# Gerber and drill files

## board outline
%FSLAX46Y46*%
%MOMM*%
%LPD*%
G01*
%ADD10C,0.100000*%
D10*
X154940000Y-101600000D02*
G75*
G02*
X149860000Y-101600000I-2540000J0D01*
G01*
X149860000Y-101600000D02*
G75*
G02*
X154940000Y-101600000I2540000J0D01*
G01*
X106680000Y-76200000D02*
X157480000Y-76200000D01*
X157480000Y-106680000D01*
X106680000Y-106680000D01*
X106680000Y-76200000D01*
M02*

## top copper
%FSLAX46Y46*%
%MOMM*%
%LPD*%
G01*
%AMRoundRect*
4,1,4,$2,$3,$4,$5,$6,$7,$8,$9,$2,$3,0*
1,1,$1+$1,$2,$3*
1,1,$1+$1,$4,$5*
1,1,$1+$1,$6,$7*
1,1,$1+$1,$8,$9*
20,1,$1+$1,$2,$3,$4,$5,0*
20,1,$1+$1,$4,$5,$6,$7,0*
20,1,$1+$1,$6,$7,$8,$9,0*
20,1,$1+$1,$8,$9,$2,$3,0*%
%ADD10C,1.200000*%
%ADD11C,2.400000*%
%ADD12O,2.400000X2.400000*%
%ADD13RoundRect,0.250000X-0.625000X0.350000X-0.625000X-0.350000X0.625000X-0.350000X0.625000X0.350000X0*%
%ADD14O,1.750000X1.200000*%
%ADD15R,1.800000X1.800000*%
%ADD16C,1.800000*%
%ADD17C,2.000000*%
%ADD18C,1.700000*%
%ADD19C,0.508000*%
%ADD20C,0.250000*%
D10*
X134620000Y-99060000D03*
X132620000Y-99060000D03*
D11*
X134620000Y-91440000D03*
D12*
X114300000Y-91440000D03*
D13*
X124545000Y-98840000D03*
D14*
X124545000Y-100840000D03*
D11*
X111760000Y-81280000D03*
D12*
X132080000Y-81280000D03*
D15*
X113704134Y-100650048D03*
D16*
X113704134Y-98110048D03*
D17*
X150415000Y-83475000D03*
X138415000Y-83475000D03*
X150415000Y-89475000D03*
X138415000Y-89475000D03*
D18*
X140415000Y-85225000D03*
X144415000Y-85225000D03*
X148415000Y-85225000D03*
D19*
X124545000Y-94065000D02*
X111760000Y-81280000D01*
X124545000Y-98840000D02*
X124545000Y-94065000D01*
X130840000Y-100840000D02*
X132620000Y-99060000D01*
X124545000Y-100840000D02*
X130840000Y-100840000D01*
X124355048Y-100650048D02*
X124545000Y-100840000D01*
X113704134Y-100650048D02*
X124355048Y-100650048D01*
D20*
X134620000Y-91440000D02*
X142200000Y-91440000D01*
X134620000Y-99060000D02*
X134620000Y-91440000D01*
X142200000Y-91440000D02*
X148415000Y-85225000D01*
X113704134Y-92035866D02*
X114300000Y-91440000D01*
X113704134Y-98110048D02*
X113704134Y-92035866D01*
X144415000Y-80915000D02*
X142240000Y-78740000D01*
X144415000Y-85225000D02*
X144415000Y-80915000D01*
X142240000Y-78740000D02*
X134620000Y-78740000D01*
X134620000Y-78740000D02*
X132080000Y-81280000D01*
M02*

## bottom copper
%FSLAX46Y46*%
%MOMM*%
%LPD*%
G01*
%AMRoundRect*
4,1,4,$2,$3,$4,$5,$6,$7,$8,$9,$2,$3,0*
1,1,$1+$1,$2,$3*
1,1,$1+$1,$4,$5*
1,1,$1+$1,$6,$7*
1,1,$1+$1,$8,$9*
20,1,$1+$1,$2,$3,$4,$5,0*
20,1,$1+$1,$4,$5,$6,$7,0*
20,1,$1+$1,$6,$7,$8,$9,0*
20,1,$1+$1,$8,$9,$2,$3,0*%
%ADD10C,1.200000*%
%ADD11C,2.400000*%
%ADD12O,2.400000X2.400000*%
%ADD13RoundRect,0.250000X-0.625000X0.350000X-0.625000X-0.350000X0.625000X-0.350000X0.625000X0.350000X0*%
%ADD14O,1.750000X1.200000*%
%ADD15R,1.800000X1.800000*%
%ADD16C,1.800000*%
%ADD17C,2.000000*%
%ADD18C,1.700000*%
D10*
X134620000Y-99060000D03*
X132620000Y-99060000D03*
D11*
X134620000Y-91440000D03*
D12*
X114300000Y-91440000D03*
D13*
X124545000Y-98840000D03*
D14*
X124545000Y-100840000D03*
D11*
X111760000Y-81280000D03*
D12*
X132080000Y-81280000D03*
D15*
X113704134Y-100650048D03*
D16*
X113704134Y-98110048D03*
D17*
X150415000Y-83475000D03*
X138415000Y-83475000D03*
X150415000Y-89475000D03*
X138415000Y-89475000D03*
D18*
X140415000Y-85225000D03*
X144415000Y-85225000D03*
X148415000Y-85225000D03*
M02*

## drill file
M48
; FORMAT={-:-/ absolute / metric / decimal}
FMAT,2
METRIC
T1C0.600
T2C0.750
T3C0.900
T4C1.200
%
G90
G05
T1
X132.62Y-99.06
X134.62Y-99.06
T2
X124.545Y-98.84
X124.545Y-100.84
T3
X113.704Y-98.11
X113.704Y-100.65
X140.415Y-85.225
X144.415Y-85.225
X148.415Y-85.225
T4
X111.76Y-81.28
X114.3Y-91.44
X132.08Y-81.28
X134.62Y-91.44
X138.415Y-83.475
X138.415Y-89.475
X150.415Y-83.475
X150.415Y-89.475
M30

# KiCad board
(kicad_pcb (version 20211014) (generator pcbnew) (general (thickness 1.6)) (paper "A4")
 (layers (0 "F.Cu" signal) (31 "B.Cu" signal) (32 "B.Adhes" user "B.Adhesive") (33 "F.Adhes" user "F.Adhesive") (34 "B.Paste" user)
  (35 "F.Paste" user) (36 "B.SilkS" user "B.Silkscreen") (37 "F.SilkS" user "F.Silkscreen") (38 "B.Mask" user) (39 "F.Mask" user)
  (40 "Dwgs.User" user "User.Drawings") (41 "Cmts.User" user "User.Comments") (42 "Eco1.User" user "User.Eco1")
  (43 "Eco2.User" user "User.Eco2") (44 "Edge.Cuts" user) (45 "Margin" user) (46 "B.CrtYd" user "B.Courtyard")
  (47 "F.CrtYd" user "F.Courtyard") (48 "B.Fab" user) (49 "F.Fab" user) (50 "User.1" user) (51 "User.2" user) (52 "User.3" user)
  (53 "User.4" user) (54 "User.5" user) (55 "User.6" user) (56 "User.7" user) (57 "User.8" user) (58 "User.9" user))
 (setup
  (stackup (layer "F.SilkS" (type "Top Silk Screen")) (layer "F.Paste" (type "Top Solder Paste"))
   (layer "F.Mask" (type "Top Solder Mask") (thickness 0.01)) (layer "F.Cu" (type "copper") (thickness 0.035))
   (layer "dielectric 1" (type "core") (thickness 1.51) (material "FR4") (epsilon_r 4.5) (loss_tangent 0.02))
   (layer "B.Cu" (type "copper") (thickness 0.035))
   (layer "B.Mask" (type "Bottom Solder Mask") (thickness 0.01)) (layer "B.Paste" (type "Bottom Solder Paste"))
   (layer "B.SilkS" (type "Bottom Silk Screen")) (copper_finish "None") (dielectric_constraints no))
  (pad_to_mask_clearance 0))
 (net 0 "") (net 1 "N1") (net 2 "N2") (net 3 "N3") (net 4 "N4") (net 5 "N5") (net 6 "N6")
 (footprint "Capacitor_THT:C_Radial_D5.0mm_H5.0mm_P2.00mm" (layer "F.Cu") (at 134.62 99.06 180)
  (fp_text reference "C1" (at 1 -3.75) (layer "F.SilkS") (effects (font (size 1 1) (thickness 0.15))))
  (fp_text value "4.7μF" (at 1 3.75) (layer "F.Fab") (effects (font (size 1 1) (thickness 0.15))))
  (pad "1" thru_hole circle (at 0 0 180) (size 1.2 1.2) (drill 0.6) (layers *.Cu *.Mask) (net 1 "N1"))
  (pad "2" thru_hole circle (at 2 0 180) (size 1.2 1.2) (drill 0.6) (layers *.Cu *.Mask) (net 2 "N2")))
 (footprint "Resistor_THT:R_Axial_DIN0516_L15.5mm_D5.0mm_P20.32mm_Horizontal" (layer "F.Cu") (at 134.62 91.44 180)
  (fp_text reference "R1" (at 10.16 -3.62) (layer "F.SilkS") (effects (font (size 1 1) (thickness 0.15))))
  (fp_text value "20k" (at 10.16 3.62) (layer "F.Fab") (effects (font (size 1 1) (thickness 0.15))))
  (pad "1" thru_hole circle (at 0 0 180) (size 2.4 2.4) (drill 1.2) (layers *.Cu *.Mask) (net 1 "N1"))
  (pad "2" thru_hole oval (at 20.32 0 180) (size 2.4 2.4) (drill 1.2) (layers *.Cu *.Mask) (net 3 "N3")))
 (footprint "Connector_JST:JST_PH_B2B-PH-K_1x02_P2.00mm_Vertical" (layer "F.Cu") (at 124.545 98.84 -90)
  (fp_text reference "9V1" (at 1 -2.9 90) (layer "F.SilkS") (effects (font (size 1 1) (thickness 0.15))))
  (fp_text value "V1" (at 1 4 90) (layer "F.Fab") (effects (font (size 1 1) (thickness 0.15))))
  (pad "1" thru_hole roundrect (at 0 0 270) (size 1.2 1.75) (drill 0.75) (layers *.Cu *.Mask) (roundrect_rratio 0.208333) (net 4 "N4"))
  (pad "2" thru_hole oval (at 2 0 270) (size 1.2 1.75) (drill 0.75) (layers *.Cu *.Mask) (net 2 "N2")))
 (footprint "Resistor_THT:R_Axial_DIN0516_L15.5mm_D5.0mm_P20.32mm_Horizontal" (layer "F.Cu") (at 111.76 81.28)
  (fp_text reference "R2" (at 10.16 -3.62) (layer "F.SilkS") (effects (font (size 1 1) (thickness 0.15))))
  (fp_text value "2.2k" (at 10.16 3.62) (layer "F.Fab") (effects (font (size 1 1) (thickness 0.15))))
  (pad "1" thru_hole circle (at 0 0) (size 2.4 2.4) (drill 1.2) (layers *.Cu *.Mask) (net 4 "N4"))
  (pad "2" thru_hole oval (at 20.32 0) (size 2.4 2.4) (drill 1.2) (layers *.Cu *.Mask) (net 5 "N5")))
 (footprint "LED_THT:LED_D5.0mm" (layer "F.Cu") (at 113.704134 100.650048 90)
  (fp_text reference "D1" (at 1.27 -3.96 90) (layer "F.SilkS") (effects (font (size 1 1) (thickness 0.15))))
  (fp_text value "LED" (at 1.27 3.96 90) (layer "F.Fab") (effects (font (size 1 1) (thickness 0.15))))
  (pad "1" thru_hole rect (at 0 0 90) (size 1.8 1.8) (drill 0.9) (layers *.Cu *.Mask) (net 2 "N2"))
  (pad "2" thru_hole circle (at 2.54 0 90) (size 1.8 1.8) (drill 0.9) (layers *.Cu *.Mask) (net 3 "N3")))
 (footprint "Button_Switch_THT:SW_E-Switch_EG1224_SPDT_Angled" (layer "F.Cu") (at 140.415 85.225)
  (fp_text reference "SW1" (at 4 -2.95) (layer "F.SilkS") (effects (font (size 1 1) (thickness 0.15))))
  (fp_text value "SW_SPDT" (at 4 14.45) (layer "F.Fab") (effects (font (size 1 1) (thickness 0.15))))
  (pad "" thru_hole circle (at 10 -1.75) (size 2 2) (drill 1.2) (layers *.Cu *.Mask))
  (pad "" thru_hole circle (at -2 -1.75) (size 2 2) (drill 1.2) (layers *.Cu *.Mask))
  (pad "" thru_hole circle (at 10 4.25) (size 2 2) (drill 1.2) (layers *.Cu *.Mask))
  (pad "" thru_hole circle (at -2 4.25) (size 2 2) (drill 1.2) (layers *.Cu *.Mask))
  (pad "1" thru_hole circle (at 0 0) (size 1.7 1.7) (drill 0.9) (layers *.Cu *.Mask) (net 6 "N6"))
  (pad "2" thru_hole circle (at 4 0) (size 1.7 1.7) (drill 0.9) (layers *.Cu *.Mask) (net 5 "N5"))
  (pad "3" thru_hole circle (at 8 0) (size 1.7 1.7) (drill 0.9) (layers *.Cu *.Mask) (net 1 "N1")))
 (gr_circle (center 152.4 101.6) (end 154.94 101.6) (layer "Edge.Cuts") (width 0.1) (fill none))
 (gr_rect (start 106.68 76.2) (end 157.48 106.68) (layer "Edge.Cuts") (width 0.1) (fill none))
 (segment (start 124.545 94.065) (end 111.76 81.28) (width 0.508) (layer "F.Cu") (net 4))
 (segment (start 124.545 98.84) (end 124.545 94.065) (width 0.508) (layer "F.Cu") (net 4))
 (segment (start 130.84 100.84) (end 132.62 99.06) (width 0.508) (layer "F.Cu") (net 2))
 (segment (start 124.545 100.84) (end 130.84 100.84) (width 0.508) (layer "F.Cu") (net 2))
 (segment (start 124.355048 100.650048) (end 124.545 100.84) (width 0.508) (layer "F.Cu") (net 2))
 (segment (start 113.704134 100.650048) (end 124.355048 100.650048) (width 0.508) (layer "F.Cu") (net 2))
 (segment (start 134.62 91.44) (end 142.2 91.44) (width 0.25) (layer "F.Cu") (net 1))
 (segment (start 134.62 99.06) (end 134.62 91.44) (width 0.25) (layer "F.Cu") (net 1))
 (segment (start 142.2 91.44) (end 148.415 85.225) (width 0.25) (layer "F.Cu") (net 1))
 (segment (start 113.704134 92.035866) (end 114.3 91.44) (width 0.25) (layer "F.Cu") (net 3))
 (segment (start 113.704134 98.110048) (end 113.704134 92.035866) (width 0.25) (layer "F.Cu") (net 3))
 (segment (start 144.415 80.915) (end 142.24 78.74) (width 0.25) (layer "F.Cu") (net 5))
 (segment (start 144.415 85.225) (end 144.415 80.915) (width 0.25) (layer "F.Cu") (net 5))
 (segment (start 142.24 78.74) (end 134.62 78.74) (width 0.25) (layer "F.Cu") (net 5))
 (segment (start 134.62 78.74) (end 132.08 81.28) (width 0.25) (layer "F.Cu") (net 5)))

